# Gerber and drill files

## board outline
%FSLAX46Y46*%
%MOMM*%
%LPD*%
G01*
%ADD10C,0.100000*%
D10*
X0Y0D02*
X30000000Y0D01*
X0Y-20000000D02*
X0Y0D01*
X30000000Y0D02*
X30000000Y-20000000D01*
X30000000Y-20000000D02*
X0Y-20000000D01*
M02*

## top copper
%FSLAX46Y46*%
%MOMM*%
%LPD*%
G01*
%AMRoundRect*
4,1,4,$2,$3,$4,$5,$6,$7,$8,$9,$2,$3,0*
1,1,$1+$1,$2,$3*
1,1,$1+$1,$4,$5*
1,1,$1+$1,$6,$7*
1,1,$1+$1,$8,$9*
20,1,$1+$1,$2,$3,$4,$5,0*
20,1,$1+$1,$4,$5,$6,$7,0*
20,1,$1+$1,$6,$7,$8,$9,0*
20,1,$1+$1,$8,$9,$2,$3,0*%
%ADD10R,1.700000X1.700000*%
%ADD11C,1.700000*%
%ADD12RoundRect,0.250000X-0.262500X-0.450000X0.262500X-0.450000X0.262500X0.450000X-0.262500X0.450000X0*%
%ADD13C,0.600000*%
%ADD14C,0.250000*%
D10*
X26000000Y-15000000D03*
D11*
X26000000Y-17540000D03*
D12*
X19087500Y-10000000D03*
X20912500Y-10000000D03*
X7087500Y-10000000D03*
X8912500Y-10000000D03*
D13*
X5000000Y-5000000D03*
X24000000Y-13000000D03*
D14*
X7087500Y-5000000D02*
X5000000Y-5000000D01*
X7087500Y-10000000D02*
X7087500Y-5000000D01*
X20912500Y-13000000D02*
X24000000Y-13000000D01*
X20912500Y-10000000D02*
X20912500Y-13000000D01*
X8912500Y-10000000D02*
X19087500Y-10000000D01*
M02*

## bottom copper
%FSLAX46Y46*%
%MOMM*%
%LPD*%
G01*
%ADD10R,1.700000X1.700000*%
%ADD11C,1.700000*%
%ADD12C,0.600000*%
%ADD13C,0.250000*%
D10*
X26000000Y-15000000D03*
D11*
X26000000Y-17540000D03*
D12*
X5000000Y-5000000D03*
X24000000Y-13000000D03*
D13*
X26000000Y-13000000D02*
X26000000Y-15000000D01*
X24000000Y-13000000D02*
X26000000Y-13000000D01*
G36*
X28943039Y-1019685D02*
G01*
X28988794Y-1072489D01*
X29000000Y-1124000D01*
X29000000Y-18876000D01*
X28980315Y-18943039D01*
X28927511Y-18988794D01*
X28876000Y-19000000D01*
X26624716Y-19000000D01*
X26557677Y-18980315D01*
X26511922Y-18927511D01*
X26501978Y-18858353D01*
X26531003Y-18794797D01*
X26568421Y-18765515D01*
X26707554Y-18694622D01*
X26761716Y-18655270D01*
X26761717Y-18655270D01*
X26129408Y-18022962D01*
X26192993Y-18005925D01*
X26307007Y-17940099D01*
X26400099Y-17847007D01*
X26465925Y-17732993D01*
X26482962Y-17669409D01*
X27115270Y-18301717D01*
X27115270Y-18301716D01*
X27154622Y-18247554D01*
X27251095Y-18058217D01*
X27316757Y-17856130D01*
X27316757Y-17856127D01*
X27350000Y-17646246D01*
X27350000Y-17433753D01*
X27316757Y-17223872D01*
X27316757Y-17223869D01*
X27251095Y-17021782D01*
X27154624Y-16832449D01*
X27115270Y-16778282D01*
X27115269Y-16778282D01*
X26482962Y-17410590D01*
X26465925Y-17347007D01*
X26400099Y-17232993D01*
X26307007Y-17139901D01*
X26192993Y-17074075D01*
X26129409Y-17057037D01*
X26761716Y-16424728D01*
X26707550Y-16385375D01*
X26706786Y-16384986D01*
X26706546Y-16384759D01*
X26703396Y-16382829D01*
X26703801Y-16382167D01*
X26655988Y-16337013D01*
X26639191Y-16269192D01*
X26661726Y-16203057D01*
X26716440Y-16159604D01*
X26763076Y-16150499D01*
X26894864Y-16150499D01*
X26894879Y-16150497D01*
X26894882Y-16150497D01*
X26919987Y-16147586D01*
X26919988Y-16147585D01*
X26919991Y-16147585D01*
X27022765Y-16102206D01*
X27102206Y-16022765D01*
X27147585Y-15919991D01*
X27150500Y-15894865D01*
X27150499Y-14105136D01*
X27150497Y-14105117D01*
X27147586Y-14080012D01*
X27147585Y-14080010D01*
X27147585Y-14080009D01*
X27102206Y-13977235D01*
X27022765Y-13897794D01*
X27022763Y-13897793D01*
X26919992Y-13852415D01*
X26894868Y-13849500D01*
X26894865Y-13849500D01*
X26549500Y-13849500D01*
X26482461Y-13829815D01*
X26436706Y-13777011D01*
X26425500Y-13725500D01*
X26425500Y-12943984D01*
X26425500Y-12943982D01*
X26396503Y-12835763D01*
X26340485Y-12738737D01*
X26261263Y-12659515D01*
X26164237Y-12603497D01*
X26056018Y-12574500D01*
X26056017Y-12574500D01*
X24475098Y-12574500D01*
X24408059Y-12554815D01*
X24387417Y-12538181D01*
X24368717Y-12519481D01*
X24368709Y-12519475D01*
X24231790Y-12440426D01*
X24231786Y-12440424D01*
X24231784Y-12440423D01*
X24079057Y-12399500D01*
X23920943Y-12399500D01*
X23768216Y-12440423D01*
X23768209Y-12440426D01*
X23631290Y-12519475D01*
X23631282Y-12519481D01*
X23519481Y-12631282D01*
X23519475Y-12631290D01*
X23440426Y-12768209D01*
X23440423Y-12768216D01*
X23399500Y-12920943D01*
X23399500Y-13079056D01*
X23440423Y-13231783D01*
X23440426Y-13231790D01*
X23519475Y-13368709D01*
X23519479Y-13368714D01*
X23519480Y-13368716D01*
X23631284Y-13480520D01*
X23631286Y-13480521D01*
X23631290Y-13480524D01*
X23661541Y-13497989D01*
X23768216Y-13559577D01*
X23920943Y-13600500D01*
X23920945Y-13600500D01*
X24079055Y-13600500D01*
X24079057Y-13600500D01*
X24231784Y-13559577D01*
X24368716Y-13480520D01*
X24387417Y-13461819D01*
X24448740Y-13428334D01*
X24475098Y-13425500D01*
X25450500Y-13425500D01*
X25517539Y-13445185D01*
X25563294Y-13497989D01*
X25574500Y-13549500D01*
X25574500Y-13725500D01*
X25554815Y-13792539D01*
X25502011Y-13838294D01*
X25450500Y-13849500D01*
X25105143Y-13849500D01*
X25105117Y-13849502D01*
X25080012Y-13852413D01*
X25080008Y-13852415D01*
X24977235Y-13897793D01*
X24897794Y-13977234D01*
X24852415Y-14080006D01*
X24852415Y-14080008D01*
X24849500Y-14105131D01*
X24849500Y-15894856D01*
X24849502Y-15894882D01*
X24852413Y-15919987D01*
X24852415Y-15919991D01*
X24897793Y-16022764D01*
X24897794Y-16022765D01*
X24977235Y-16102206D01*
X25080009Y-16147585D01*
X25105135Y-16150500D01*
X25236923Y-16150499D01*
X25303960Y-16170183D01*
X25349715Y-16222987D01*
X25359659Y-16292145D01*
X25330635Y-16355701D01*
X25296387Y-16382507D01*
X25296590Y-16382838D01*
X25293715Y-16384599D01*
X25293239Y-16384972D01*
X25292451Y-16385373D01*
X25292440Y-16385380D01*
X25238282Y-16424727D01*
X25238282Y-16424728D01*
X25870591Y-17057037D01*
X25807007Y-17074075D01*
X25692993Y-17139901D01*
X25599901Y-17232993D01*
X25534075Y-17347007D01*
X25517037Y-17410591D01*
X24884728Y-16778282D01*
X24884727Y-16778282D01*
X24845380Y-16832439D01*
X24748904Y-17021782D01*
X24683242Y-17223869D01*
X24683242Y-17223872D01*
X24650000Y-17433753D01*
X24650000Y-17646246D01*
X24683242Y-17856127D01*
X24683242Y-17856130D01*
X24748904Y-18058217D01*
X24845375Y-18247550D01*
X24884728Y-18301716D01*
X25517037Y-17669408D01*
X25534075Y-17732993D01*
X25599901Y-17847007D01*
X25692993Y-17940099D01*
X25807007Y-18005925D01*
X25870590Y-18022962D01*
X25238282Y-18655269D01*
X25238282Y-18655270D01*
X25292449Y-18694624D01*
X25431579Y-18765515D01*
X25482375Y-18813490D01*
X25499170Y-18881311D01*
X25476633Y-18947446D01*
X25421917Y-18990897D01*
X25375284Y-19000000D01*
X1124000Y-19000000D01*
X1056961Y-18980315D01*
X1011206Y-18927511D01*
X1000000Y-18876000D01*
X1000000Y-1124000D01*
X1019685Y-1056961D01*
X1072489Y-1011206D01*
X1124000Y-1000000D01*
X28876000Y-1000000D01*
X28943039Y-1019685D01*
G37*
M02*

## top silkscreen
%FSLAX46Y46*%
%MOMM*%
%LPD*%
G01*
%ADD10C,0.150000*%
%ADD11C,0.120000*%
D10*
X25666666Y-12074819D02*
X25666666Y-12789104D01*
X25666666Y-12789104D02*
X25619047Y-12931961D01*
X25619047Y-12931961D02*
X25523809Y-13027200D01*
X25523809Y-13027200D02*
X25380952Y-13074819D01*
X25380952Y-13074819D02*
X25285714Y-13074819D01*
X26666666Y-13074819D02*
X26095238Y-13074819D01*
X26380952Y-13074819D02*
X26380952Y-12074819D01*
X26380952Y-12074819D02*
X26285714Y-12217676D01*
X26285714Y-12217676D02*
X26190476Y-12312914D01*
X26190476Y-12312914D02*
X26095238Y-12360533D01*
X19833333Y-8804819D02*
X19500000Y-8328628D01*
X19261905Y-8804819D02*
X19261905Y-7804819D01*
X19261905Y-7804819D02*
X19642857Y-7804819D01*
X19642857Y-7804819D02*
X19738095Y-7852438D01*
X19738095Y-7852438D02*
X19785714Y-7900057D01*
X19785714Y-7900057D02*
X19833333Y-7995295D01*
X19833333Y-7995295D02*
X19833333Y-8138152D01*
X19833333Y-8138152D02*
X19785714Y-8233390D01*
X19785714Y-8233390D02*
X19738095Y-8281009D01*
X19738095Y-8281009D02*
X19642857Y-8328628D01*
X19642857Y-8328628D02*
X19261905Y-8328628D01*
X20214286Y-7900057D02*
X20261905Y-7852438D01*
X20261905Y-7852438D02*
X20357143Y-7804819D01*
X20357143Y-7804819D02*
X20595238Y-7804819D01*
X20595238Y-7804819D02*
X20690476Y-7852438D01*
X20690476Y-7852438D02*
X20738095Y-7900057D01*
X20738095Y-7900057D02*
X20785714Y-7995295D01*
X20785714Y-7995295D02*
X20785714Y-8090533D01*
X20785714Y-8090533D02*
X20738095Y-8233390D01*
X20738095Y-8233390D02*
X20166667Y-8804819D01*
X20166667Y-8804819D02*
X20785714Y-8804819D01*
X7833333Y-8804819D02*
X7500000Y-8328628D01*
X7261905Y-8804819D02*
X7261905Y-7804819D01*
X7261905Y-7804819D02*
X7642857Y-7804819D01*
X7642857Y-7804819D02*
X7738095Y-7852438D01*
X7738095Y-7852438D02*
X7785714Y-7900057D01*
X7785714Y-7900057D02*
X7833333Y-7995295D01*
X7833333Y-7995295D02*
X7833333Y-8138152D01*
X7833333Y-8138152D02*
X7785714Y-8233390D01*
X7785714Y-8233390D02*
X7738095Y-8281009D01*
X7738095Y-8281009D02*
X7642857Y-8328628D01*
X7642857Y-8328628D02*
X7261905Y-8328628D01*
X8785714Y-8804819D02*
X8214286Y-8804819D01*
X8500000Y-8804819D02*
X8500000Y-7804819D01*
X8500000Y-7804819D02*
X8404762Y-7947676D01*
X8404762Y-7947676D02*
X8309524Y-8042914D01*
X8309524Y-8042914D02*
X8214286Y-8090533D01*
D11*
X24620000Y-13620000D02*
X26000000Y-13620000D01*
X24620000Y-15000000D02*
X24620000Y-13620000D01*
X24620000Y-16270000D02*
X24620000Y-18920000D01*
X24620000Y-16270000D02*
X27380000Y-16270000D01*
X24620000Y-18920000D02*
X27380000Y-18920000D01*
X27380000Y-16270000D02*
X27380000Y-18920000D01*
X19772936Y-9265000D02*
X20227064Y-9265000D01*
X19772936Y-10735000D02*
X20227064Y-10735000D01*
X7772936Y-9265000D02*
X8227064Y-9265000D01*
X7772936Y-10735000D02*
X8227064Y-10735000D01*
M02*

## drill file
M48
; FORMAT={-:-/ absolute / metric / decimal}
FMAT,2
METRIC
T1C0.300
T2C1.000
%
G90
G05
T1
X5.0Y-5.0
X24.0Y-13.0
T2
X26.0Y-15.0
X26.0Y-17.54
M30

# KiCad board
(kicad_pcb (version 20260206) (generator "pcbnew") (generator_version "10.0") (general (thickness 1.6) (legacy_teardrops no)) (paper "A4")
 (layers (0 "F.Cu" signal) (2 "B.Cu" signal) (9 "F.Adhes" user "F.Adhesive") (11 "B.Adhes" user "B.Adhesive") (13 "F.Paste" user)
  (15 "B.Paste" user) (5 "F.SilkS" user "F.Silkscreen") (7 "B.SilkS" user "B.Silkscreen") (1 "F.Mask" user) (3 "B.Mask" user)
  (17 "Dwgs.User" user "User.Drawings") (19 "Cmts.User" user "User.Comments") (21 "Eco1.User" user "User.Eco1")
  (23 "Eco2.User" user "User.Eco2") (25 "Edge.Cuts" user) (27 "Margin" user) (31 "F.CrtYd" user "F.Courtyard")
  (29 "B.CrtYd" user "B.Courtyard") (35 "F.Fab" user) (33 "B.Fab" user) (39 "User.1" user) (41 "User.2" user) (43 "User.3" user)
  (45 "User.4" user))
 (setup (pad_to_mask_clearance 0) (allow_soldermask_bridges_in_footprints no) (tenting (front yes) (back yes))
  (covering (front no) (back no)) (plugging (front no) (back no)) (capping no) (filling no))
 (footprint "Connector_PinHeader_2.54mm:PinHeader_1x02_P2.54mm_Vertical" (layer "F.Cu") (at 26 15)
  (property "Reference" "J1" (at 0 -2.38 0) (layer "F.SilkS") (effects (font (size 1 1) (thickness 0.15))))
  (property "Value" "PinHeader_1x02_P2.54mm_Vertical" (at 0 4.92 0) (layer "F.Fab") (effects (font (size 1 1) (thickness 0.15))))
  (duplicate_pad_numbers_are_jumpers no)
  (fp_line (start -1.38 -1.38) (end 0 -1.38) (stroke (width 0.12) (type solid)) (layer "F.SilkS"))
  (fp_line (start -1.38 0) (end -1.38 -1.38) (stroke (width 0.12) (type solid)) (layer "F.SilkS"))
  (fp_line (start -1.38 1.27) (end -1.38 3.92) (stroke (width 0.12) (type solid)) (layer "F.SilkS"))
  (fp_line (start -1.38 1.27) (end 1.38 1.27) (stroke (width 0.12) (type solid)) (layer "F.SilkS"))
  (fp_line (start -1.38 3.92) (end 1.38 3.92) (stroke (width 0.12) (type solid)) (layer "F.SilkS"))
  (fp_line (start 1.38 1.27) (end 1.38 3.92) (stroke (width 0.12) (type solid)) (layer "F.SilkS"))
  (pad "1" thru_hole rect (at 0 0) (size 1.7 1.7) (drill 1) (layers "*.Cu" "*.Mask") (remove_unused_layers no) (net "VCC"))
  (pad "2" thru_hole circle (at 0 2.54) (size 1.7 1.7) (drill 1) (layers "*.Cu" "*.Mask") (remove_unused_layers no) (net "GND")))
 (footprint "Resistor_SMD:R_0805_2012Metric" (layer "F.Cu") (at 20 10)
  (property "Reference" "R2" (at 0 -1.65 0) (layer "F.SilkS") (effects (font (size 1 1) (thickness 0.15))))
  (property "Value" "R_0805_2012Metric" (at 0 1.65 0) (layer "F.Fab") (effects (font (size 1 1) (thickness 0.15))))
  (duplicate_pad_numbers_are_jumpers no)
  (fp_line (start -0.227064 -0.735) (end 0.227064 -0.735) (stroke (width 0.12) (type solid)) (layer "F.SilkS"))
  (fp_line (start -0.227064 0.735) (end 0.227064 0.735) (stroke (width 0.12) (type solid)) (layer "F.SilkS"))
  (pad "1" smd roundrect (at -0.9125 0) (size 1.025 1.4) (layers "F.Cu" "F.Mask" "F.Paste") (roundrect_rratio 0.243902) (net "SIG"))
  (pad "2" smd roundrect (at 0.9125 0) (size 1.025 1.4) (layers "F.Cu" "F.Mask" "F.Paste") (roundrect_rratio 0.243902) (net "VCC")))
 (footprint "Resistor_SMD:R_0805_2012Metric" (layer "F.Cu") (at 8 10)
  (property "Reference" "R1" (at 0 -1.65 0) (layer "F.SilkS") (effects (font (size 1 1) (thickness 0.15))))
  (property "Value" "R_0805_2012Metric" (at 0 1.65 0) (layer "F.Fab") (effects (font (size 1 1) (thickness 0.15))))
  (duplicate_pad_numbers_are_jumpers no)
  (fp_line (start -0.227064 -0.735) (end 0.227064 -0.735) (stroke (width 0.12) (type solid)) (layer "F.SilkS"))
  (fp_line (start -0.227064 0.735) (end 0.227064 0.735) (stroke (width 0.12) (type solid)) (layer "F.SilkS"))
  (pad "1" smd roundrect (at -0.9125 0) (size 1.025 1.4) (layers "F.Cu" "F.Mask" "F.Paste") (roundrect_rratio 0.243902) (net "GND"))
  (pad "2" smd roundrect (at 0.9125 0) (size 1.025 1.4) (layers "F.Cu" "F.Mask" "F.Paste") (roundrect_rratio 0.243902) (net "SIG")))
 (gr_line (start 0 0) (end 30 0) (stroke (width 0.1) (type default)) (layer "Edge.Cuts"))
 (gr_line (start 0 20) (end 0 0) (stroke (width 0.1) (type default)) (layer "Edge.Cuts"))
 (gr_line (start 30 0) (end 30 20) (stroke (width 0.1) (type default)) (layer "Edge.Cuts"))
 (gr_line (start 30 20) (end 0 20) (stroke (width 0.1) (type default)) (layer "Edge.Cuts"))
 (segment (start 7.0875 5) (end 5 5) (width 0.25) (layer "F.Cu") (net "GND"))
 (segment (start 7.0875 10) (end 7.0875 5) (width 0.25) (layer "F.Cu") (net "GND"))
 (via (at 5 5) (size 0.6) (drill 0.3) (layers "F.Cu" "B.Cu") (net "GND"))
 (segment (start 20.9125 13) (end 24 13) (width 0.25) (layer "F.Cu") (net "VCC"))
 (segment (start 20.9125 10) (end 20.9125 13) (width 0.25) (layer "F.Cu") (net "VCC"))
 (via (at 24 13) (size 0.6) (drill 0.3) (layers "F.Cu" "B.Cu") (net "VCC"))
 (segment (start 26 13) (end 26 15) (width 0.25) (layer "B.Cu") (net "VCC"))
 (segment (start 24 13) (end 26 13) (width 0.25) (layer "B.Cu") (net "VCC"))
 (segment (start 8.9125 10) (end 19.0875 10) (width 0.25) (layer "F.Cu") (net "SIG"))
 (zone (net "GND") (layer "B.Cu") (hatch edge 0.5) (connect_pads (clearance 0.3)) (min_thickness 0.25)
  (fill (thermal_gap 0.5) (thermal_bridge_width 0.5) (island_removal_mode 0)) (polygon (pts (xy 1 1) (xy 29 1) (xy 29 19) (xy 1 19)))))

